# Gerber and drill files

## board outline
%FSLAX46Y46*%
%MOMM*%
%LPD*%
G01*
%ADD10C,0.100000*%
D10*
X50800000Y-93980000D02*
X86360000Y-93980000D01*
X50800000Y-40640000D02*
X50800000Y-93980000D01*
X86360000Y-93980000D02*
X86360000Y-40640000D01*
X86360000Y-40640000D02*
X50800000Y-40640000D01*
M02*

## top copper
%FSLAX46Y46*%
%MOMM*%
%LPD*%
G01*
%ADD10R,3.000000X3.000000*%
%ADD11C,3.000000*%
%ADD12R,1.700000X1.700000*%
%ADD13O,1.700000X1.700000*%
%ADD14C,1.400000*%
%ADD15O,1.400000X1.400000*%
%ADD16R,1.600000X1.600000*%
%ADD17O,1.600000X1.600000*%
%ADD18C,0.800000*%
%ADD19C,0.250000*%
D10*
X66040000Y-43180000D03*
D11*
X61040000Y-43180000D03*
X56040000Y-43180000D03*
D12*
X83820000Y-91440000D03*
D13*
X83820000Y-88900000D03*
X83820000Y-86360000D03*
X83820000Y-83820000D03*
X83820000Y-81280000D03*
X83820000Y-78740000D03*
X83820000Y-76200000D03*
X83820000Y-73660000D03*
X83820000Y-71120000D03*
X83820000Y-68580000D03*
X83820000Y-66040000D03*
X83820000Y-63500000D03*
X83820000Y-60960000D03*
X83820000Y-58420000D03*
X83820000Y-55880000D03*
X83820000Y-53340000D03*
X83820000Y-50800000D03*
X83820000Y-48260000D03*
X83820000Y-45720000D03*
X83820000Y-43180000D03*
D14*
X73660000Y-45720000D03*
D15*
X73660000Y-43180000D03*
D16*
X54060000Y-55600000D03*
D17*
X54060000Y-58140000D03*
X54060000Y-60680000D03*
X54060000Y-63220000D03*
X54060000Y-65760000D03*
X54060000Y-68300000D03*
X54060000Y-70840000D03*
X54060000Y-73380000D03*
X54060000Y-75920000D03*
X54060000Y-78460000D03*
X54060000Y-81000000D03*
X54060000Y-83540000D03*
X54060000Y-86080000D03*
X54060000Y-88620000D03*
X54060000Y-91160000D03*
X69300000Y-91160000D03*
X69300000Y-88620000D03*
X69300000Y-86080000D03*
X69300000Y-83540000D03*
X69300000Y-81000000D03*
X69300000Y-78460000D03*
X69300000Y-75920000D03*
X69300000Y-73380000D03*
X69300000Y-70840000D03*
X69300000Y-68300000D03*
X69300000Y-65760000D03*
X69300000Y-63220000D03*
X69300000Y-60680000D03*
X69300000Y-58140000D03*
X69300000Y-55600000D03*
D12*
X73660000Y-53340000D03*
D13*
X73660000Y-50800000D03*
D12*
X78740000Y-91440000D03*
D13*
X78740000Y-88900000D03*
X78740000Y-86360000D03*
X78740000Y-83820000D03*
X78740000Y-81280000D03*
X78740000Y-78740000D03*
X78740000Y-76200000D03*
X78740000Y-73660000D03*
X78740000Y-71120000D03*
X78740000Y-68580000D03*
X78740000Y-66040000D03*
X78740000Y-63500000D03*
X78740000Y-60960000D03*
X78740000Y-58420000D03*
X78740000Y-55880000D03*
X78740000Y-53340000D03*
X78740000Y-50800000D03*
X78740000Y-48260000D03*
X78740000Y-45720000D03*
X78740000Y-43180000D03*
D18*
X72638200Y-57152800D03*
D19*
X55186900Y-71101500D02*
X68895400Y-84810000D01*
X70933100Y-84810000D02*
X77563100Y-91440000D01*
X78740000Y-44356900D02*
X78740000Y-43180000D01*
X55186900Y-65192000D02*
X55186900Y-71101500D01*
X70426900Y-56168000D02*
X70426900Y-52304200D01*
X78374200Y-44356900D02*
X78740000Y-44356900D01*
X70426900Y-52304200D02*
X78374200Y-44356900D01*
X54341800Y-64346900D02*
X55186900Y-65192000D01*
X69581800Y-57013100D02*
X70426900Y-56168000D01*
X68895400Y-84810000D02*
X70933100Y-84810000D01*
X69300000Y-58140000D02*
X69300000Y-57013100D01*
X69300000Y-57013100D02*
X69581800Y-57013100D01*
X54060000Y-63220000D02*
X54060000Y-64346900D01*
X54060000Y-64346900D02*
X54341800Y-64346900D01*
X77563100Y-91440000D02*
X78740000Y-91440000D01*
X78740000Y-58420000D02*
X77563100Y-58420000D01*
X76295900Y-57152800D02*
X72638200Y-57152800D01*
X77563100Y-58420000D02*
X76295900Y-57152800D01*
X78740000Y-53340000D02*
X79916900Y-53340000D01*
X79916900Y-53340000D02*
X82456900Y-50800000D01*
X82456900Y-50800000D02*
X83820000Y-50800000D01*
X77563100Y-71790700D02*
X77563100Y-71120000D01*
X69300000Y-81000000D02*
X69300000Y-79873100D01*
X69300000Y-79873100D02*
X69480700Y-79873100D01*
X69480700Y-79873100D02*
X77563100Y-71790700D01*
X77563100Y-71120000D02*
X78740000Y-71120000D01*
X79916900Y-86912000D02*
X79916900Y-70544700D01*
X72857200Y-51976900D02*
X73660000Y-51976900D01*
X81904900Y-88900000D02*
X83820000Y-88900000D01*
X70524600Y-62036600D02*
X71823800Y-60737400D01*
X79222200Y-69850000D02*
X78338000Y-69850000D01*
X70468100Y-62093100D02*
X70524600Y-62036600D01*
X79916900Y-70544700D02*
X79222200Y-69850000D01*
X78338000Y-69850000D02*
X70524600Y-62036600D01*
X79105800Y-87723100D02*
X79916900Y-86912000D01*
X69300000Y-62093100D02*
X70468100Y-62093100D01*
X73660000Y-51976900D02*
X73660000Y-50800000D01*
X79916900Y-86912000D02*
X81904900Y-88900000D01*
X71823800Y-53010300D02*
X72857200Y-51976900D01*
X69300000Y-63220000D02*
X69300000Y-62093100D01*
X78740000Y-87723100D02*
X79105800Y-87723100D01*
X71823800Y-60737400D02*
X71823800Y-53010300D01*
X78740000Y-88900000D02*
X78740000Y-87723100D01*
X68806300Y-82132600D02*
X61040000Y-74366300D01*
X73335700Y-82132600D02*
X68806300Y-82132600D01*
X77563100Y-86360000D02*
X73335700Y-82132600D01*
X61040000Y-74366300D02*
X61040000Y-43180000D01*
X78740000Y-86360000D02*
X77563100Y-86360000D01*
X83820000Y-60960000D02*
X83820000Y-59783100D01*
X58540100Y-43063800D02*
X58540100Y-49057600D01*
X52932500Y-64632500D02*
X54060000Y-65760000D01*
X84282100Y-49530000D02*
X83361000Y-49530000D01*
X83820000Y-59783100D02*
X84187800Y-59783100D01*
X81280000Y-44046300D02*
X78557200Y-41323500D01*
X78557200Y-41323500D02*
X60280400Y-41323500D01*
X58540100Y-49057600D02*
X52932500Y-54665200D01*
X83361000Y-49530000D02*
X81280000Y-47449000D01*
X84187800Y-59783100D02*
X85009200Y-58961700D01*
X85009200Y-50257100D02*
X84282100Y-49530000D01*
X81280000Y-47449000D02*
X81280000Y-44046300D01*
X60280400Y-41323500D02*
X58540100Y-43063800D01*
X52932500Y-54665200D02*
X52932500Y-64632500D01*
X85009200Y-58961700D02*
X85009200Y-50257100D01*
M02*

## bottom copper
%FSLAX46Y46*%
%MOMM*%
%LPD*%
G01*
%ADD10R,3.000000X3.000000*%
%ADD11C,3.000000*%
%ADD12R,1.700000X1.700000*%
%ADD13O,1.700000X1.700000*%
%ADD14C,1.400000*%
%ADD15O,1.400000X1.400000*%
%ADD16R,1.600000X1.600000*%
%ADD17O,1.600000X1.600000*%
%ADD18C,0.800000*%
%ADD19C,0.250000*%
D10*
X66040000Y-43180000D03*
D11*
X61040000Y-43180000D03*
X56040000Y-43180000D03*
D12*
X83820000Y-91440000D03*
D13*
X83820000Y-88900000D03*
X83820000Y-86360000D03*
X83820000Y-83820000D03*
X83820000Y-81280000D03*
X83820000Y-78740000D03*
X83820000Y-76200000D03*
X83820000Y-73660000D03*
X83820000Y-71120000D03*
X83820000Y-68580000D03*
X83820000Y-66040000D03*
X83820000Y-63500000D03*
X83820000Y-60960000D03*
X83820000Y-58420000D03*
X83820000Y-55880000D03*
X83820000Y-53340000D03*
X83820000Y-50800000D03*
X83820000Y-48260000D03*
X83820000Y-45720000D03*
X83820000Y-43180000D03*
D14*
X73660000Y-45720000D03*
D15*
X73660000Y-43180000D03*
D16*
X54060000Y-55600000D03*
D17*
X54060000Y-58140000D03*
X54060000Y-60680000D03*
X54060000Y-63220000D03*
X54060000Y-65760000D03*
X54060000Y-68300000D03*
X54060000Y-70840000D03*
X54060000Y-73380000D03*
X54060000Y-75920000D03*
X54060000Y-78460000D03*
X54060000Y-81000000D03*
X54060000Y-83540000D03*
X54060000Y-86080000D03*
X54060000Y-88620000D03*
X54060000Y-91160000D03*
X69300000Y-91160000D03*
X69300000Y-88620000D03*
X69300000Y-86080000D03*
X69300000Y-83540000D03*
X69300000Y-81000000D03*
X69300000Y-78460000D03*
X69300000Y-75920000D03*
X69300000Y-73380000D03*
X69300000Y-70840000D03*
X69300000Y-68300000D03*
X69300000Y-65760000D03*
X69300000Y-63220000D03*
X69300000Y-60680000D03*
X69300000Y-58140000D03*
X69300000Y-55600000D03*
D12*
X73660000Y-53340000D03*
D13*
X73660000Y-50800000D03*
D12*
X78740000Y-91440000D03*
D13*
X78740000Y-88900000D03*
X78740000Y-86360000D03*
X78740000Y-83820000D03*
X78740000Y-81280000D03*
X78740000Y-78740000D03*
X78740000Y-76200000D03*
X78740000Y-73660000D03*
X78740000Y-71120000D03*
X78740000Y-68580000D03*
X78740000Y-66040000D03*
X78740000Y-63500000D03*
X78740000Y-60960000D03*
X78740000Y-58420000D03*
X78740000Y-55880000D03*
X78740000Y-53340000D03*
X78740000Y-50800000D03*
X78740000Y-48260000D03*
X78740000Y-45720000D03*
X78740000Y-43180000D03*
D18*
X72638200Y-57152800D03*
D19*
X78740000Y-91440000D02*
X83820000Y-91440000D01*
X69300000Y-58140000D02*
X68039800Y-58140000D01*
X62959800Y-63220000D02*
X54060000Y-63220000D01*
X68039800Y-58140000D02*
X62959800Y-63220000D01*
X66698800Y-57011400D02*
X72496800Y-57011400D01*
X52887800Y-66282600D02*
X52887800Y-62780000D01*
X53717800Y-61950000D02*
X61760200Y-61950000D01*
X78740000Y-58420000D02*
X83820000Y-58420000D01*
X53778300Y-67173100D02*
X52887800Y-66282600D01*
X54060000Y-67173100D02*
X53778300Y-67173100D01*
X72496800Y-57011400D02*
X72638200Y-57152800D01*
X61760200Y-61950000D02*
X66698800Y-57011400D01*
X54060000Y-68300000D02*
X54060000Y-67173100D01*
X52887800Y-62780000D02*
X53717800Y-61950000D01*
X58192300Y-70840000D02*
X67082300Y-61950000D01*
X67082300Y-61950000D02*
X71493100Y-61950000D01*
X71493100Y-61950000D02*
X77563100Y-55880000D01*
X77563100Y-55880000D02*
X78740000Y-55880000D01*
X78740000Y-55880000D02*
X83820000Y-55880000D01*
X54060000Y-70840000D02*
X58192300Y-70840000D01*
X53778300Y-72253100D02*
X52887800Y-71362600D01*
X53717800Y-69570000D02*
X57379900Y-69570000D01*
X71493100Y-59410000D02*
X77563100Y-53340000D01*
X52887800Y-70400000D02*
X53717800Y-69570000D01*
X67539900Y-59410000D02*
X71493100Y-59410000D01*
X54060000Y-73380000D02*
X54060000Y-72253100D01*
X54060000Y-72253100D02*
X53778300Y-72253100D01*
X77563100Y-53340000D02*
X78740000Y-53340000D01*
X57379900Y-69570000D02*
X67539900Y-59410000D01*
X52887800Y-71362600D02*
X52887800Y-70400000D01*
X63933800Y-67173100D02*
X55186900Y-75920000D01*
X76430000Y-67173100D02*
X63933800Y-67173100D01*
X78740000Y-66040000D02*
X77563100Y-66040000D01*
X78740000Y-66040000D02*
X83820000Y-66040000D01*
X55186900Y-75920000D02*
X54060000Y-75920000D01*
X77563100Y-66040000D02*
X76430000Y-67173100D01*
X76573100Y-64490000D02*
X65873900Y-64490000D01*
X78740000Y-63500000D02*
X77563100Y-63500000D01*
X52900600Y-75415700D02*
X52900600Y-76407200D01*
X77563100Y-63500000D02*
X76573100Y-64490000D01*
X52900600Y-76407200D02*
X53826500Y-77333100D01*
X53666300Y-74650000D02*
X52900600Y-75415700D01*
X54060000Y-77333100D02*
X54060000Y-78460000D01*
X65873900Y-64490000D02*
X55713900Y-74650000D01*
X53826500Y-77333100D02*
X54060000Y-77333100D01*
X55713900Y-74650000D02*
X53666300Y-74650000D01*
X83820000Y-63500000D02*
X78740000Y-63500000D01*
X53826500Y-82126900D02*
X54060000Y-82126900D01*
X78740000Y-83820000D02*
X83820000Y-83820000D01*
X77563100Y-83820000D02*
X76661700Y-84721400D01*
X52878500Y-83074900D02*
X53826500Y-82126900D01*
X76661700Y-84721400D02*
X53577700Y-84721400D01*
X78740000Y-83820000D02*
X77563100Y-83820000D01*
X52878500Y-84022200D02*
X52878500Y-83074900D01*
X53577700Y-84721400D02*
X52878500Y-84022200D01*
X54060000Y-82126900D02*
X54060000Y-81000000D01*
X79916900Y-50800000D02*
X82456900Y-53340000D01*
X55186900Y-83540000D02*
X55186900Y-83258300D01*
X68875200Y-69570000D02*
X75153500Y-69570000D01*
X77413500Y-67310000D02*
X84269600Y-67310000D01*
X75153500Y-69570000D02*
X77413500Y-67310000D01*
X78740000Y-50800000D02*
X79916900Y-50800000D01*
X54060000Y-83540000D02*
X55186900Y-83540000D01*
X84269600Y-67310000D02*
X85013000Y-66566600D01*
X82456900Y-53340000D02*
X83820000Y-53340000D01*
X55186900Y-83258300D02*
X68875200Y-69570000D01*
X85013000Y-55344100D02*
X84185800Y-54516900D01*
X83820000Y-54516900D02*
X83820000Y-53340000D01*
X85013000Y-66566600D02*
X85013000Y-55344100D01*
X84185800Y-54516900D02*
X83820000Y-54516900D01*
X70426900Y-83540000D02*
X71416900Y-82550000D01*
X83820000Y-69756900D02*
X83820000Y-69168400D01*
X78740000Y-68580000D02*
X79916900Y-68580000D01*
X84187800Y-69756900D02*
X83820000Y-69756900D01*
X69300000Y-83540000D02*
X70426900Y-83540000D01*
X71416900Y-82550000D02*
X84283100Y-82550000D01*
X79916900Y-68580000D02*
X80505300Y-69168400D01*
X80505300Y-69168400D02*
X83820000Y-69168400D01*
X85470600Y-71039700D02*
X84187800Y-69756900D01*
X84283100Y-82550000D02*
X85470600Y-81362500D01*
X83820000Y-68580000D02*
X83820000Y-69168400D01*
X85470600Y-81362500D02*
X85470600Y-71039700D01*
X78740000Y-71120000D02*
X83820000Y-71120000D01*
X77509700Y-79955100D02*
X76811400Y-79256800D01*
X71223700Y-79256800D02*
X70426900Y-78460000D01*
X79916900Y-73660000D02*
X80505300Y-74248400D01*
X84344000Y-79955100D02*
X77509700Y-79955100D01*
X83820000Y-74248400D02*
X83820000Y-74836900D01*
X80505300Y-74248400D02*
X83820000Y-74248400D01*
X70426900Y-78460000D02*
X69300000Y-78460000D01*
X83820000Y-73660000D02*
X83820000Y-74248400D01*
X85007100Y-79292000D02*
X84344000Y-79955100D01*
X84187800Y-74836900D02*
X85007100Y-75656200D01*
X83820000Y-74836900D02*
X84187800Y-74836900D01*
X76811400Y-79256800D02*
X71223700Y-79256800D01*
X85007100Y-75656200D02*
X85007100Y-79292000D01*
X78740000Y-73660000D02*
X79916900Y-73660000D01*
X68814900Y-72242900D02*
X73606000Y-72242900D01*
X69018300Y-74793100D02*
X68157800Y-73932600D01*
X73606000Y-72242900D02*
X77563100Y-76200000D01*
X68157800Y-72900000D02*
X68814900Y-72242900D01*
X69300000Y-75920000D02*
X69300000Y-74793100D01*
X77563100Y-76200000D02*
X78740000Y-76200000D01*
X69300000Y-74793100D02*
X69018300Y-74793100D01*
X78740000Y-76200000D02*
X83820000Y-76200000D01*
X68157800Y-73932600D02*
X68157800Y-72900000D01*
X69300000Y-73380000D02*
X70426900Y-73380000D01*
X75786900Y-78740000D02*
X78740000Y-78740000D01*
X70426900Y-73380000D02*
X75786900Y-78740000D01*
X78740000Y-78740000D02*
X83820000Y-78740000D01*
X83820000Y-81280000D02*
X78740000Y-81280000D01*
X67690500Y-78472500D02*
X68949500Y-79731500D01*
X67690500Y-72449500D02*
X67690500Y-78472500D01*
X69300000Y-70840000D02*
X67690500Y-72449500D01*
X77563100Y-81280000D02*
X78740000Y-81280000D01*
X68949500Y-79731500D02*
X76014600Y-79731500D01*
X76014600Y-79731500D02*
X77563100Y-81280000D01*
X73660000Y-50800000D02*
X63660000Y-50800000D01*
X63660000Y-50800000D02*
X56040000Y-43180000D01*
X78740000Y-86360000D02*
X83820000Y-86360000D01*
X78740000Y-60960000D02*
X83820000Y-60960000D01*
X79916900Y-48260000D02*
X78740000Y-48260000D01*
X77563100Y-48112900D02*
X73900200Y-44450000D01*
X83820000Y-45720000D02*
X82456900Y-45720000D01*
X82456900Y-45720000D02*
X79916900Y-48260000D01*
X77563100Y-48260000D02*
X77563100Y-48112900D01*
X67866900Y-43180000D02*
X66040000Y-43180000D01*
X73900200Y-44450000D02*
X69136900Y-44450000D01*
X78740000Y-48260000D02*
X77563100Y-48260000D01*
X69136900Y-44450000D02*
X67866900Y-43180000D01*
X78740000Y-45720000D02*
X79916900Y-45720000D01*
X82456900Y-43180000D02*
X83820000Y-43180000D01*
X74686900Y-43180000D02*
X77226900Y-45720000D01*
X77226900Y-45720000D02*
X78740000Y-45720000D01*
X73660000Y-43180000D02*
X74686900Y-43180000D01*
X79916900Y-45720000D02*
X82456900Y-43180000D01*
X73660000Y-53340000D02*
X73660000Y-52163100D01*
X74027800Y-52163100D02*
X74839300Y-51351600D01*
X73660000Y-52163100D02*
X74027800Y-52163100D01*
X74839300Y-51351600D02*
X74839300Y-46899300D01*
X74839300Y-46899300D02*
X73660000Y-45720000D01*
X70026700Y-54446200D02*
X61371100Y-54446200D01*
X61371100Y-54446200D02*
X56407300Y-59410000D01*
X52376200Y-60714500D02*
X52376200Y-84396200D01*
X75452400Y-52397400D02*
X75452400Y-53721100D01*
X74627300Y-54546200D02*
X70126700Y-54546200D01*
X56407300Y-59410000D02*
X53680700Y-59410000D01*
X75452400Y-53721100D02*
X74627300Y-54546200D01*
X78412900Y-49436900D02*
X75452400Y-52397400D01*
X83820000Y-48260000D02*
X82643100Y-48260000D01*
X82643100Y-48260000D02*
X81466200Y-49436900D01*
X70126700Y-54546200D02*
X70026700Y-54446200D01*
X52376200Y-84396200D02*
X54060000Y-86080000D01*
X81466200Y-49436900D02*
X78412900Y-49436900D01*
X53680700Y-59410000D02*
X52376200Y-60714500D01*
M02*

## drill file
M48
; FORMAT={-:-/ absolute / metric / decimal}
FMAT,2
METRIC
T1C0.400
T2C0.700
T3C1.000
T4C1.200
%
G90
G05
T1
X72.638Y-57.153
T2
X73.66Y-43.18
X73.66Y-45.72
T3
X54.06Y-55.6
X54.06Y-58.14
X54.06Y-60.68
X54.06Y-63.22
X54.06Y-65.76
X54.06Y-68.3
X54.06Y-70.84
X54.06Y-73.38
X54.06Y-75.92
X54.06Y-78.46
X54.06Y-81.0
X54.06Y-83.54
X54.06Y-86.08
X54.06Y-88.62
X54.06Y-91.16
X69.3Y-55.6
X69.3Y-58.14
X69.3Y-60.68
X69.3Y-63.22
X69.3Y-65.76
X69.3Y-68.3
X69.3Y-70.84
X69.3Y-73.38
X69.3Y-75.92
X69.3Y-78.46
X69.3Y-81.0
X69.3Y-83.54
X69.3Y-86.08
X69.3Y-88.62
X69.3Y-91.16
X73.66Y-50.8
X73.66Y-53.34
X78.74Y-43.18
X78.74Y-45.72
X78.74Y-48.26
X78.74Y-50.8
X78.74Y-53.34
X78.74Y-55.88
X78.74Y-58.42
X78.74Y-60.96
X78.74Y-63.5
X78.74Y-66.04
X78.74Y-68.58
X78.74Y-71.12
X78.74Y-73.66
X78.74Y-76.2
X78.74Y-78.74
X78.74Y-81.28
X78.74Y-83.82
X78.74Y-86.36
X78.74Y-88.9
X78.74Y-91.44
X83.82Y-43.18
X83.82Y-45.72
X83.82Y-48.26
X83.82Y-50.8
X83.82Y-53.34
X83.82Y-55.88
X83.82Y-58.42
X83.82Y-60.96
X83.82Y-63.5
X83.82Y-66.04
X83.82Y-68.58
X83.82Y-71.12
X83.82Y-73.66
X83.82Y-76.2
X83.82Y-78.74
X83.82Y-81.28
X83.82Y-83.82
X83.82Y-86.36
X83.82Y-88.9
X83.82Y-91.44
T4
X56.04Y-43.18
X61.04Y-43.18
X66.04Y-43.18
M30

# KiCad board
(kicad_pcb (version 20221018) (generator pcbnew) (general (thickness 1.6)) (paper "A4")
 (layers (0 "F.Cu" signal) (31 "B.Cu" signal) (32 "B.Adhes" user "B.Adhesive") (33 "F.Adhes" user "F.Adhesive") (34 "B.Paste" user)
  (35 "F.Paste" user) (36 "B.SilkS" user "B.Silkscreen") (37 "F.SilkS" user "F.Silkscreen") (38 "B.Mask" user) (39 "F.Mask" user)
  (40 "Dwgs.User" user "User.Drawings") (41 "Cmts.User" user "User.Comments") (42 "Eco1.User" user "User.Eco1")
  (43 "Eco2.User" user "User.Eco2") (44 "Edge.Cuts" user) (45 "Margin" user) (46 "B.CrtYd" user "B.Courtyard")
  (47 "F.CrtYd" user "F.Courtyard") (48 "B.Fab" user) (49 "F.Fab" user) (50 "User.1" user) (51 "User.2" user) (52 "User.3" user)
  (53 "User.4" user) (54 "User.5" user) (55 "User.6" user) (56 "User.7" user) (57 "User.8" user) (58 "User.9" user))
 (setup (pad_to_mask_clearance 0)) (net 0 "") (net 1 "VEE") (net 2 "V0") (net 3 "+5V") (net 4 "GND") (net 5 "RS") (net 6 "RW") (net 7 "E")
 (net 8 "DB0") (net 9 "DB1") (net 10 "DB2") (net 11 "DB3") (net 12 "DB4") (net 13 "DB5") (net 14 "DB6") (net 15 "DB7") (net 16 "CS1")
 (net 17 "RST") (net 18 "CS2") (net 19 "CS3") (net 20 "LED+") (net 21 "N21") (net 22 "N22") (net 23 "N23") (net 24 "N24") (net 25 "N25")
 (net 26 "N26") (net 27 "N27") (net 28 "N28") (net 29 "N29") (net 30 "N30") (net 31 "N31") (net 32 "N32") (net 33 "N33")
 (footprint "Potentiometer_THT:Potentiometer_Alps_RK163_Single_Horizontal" (layer "F.Cu") (at 66.04 43.18 -90)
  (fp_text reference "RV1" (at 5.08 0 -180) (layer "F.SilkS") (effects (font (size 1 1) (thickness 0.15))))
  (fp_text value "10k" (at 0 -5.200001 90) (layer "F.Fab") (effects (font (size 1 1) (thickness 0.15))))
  (pad "1" thru_hole rect (at 0 0 90) (size 3 3) (drill 1.2) (layers "*.Cu" "*.Mask") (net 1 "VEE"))
  (pad "2" thru_hole circle (at 0 5 90) (size 3 3) (drill 1.2) (layers "*.Cu" "*.Mask") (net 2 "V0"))
  (pad "3" thru_hole circle (at 0 10 90) (size 3 3) (drill 1.2) (layers "*.Cu" "*.Mask") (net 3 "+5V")))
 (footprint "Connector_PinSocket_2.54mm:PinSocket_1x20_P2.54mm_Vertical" (layer "F.Cu") (at 83.82 91.44 180)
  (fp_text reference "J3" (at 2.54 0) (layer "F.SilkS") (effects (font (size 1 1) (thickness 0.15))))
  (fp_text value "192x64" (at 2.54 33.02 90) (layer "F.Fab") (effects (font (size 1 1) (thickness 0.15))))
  (pad "1" thru_hole rect (at 0 0 180) (size 1.7 1.7) (drill 1) (layers "*.Cu" "*.Mask") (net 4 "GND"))
  (pad "2" thru_hole oval (at 0 2.54 180) (size 1.7 1.7) (drill 1) (layers "*.Cu" "*.Mask") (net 3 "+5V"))
  (pad "3" thru_hole oval (at 0 5.08 180) (size 1.7 1.7) (drill 1) (layers "*.Cu" "*.Mask") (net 2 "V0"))
  (pad "4" thru_hole oval (at 0 7.62 180) (size 1.7 1.7) (drill 1) (layers "*.Cu" "*.Mask") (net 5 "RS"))
  (pad "5" thru_hole oval (at 0 10.16 180) (size 1.7 1.7) (drill 1) (layers "*.Cu" "*.Mask") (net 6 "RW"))
  (pad "6" thru_hole oval (at 0 12.7 180) (size 1.7 1.7) (drill 1) (layers "*.Cu" "*.Mask") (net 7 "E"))
  (pad "7" thru_hole oval (at 0 15.24 180) (size 1.7 1.7) (drill 1) (layers "*.Cu" "*.Mask") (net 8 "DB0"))
  (pad "8" thru_hole oval (at 0 17.78 180) (size 1.7 1.7) (drill 1) (layers "*.Cu" "*.Mask") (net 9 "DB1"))
  (pad "9" thru_hole oval (at 0 20.32 180) (size 1.7 1.7) (drill 1) (layers "*.Cu" "*.Mask") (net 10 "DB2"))
  (pad "10" thru_hole oval (at 0 22.86 180) (size 1.7 1.7) (drill 1) (layers "*.Cu" "*.Mask") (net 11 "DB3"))
  (pad "11" thru_hole oval (at 0 25.4 180) (size 1.7 1.7) (drill 1) (layers "*.Cu" "*.Mask") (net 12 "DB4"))
  (pad "12" thru_hole oval (at 0 27.94 180) (size 1.7 1.7) (drill 1) (layers "*.Cu" "*.Mask") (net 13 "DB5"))
  (pad "13" thru_hole oval (at 0 30.48 180) (size 1.7 1.7) (drill 1) (layers "*.Cu" "*.Mask") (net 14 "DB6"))
  (pad "14" thru_hole oval (at 0 33.02 180) (size 1.7 1.7) (drill 1) (layers "*.Cu" "*.Mask") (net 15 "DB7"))
  (pad "15" thru_hole oval (at 0 35.56 180) (size 1.7 1.7) (drill 1) (layers "*.Cu" "*.Mask") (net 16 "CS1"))
  (pad "16" thru_hole oval (at 0 38.1 180) (size 1.7 1.7) (drill 1) (layers "*.Cu" "*.Mask") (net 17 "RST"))
  (pad "17" thru_hole oval (at 0 40.64 180) (size 1.7 1.7) (drill 1) (layers "*.Cu" "*.Mask") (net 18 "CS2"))
  (pad "18" thru_hole oval (at 0 43.18 180) (size 1.7 1.7) (drill 1) (layers "*.Cu" "*.Mask") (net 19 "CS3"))
  (pad "19" thru_hole oval (at 0 45.72 180) (size 1.7 1.7) (drill 1) (layers "*.Cu" "*.Mask") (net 1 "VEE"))
  (pad "20" thru_hole oval (at 0 48.26 180) (size 1.7 1.7) (drill 1) (layers "*.Cu" "*.Mask") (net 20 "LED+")))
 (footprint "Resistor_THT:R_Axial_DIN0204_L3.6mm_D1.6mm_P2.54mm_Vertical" (layer "F.Cu") (at 73.66 45.72 90)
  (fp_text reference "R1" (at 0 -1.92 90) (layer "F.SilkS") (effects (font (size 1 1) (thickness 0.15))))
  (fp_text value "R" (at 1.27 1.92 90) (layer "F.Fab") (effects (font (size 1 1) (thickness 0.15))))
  (pad "1" thru_hole circle (at 0 0 90) (size 1.4 1.4) (drill 0.7) (layers "*.Cu" "*.Mask") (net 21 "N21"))
  (pad "2" thru_hole oval (at 2.54 0 90) (size 1.4 1.4) (drill 0.7) (layers "*.Cu" "*.Mask") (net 20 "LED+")))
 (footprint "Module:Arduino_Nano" (layer "F.Cu") (at 54.06 55.6)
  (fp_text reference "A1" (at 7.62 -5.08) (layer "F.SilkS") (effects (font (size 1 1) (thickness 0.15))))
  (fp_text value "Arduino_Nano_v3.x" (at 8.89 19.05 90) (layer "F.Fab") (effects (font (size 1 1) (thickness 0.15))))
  (pad "1" thru_hole rect (at 0 0) (size 1.6 1.6) (drill 1) (layers "*.Cu" "*.Mask") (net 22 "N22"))
  (pad "2" thru_hole oval (at 0 2.54) (size 1.6 1.6) (drill 1) (layers "*.Cu" "*.Mask") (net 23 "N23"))
  (pad "3" thru_hole oval (at 0 5.08) (size 1.6 1.6) (drill 1) (layers "*.Cu" "*.Mask") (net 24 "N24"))
  (pad "4" thru_hole oval (at 0 7.62) (size 1.6 1.6) (drill 1) (layers "*.Cu" "*.Mask") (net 4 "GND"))
  (pad "5" thru_hole oval (at 0 10.16) (size 1.6 1.6) (drill 1) (layers "*.Cu" "*.Mask") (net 14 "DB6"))
  (pad "6" thru_hole oval (at 0 12.7) (size 1.6 1.6) (drill 1) (layers "*.Cu" "*.Mask") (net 15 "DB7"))
  (pad "7" thru_hole oval (at 0 15.24) (size 1.6 1.6) (drill 1) (layers "*.Cu" "*.Mask") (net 16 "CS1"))
  (pad "8" thru_hole oval (at 0 17.78) (size 1.6 1.6) (drill 1) (layers "*.Cu" "*.Mask") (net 18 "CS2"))
  (pad "9" thru_hole oval (at 0 20.32) (size 1.6 1.6) (drill 1) (layers "*.Cu" "*.Mask") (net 12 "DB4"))
  (pad "10" thru_hole oval (at 0 22.86) (size 1.6 1.6) (drill 1) (layers "*.Cu" "*.Mask") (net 13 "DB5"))
  (pad "11" thru_hole oval (at 0 25.4) (size 1.6 1.6) (drill 1) (layers "*.Cu" "*.Mask") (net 5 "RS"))
  (pad "12" thru_hole oval (at 0 27.94) (size 1.6 1.6) (drill 1) (layers "*.Cu" "*.Mask") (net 17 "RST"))
  (pad "13" thru_hole oval (at 0 30.48) (size 1.6 1.6) (drill 1) (layers "*.Cu" "*.Mask") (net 19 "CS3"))
  (pad "14" thru_hole oval (at 0 33.02) (size 1.6 1.6) (drill 1) (layers "*.Cu" "*.Mask") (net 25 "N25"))
  (pad "15" thru_hole oval (at 0 35.56) (size 1.6 1.6) (drill 1) (layers "*.Cu" "*.Mask") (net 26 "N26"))
  (pad "16" thru_hole oval (at 15.24 35.56) (size 1.6 1.6) (drill 1) (layers "*.Cu" "*.Mask") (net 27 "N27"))
  (pad "17" thru_hole oval (at 15.24 33.02) (size 1.6 1.6) (drill 1) (layers "*.Cu" "*.Mask") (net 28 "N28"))
  (pad "18" thru_hole oval (at 15.24 30.48) (size 1.6 1.6) (drill 1) (layers "*.Cu" "*.Mask") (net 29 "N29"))
  (pad "19" thru_hole oval (at 15.24 27.94) (size 1.6 1.6) (drill 1) (layers "*.Cu" "*.Mask") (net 11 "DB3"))
  (pad "20" thru_hole oval (at 15.24 25.4) (size 1.6 1.6) (drill 1) (layers "*.Cu" "*.Mask") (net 10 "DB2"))
  (pad "21" thru_hole oval (at 15.24 22.86) (size 1.6 1.6) (drill 1) (layers "*.Cu" "*.Mask") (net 9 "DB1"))
  (pad "22" thru_hole oval (at 15.24 20.32) (size 1.6 1.6) (drill 1) (layers "*.Cu" "*.Mask") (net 8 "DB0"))
  (pad "23" thru_hole oval (at 15.24 17.78) (size 1.6 1.6) (drill 1) (layers "*.Cu" "*.Mask") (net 7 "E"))
  (pad "24" thru_hole oval (at 15.24 15.24) (size 1.6 1.6) (drill 1) (layers "*.Cu" "*.Mask") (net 6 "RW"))
  (pad "25" thru_hole oval (at 15.24 12.7) (size 1.6 1.6) (drill 1) (layers "*.Cu" "*.Mask") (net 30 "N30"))
  (pad "26" thru_hole oval (at 15.24 10.16) (size 1.6 1.6) (drill 1) (layers "*.Cu" "*.Mask") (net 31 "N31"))
  (pad "27" thru_hole oval (at 15.24 7.62) (size 1.6 1.6) (drill 1) (layers "*.Cu" "*.Mask") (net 3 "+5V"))
  (pad "28" thru_hole oval (at 15.24 5.08) (size 1.6 1.6) (drill 1) (layers "*.Cu" "*.Mask") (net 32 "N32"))
  (pad "29" thru_hole oval (at 15.24 2.54) (size 1.6 1.6) (drill 1) (layers "*.Cu" "*.Mask") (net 4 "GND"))
  (pad "30" thru_hole oval (at 15.24 0) (size 1.6 1.6) (drill 1) (layers "*.Cu" "*.Mask") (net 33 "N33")))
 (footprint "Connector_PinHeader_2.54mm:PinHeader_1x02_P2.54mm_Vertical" (layer "F.Cu") (at 73.66 53.34 180)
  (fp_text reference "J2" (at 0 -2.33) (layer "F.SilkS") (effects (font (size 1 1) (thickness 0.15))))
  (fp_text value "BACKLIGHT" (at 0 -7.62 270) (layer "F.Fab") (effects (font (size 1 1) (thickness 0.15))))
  (pad "1" thru_hole rect (at 0 0 180) (size 1.7 1.7) (drill 1) (layers "*.Cu" "*.Mask") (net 21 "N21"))
  (pad "2" thru_hole oval (at 0 2.54 180) (size 1.7 1.7) (drill 1) (layers "*.Cu" "*.Mask") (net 3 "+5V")))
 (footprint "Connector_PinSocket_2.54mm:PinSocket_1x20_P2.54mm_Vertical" (layer "F.Cu") (at 78.74 91.44 180)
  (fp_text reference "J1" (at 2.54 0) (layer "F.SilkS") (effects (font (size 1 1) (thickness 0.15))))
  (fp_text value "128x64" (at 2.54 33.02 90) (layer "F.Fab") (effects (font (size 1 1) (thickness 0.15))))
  (pad "1" thru_hole rect (at 0 0 180) (size 1.7 1.7) (drill 1) (layers "*.Cu" "*.Mask") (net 4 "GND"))
  (pad "2" thru_hole oval (at 0 2.54 180) (size 1.7 1.7) (drill 1) (layers "*.Cu" "*.Mask") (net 3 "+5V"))
  (pad "3" thru_hole oval (at 0 5.08 180) (size 1.7 1.7) (drill 1) (layers "*.Cu" "*.Mask") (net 2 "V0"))
  (pad "4" thru_hole oval (at 0 7.62 180) (size 1.7 1.7) (drill 1) (layers "*.Cu" "*.Mask") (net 5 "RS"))
  (pad "5" thru_hole oval (at 0 10.16 180) (size 1.7 1.7) (drill 1) (layers "*.Cu" "*.Mask") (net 6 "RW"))
  (pad "6" thru_hole oval (at 0 12.7 180) (size 1.7 1.7) (drill 1) (layers "*.Cu" "*.Mask") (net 7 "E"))
  (pad "7" thru_hole oval (at 0 15.24 180) (size 1.7 1.7) (drill 1) (layers "*.Cu" "*.Mask") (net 8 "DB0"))
  (pad "8" thru_hole oval (at 0 17.78 180) (size 1.7 1.7) (drill 1) (layers "*.Cu" "*.Mask") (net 9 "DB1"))
  (pad "9" thru_hole oval (at 0 20.32 180) (size 1.7 1.7) (drill 1) (layers "*.Cu" "*.Mask") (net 10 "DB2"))
  (pad "10" thru_hole oval (at 0 22.86 180) (size 1.7 1.7) (drill 1) (layers "*.Cu" "*.Mask") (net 11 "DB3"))
  (pad "11" thru_hole oval (at 0 25.4 180) (size 1.7 1.7) (drill 1) (layers "*.Cu" "*.Mask") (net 12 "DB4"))
  (pad "12" thru_hole oval (at 0 27.94 180) (size 1.7 1.7) (drill 1) (layers "*.Cu" "*.Mask") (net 13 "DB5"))
  (pad "13" thru_hole oval (at 0 30.48 180) (size 1.7 1.7) (drill 1) (layers "*.Cu" "*.Mask") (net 14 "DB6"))
  (pad "14" thru_hole oval (at 0 33.02 180) (size 1.7 1.7) (drill 1) (layers "*.Cu" "*.Mask") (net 15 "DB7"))
  (pad "15" thru_hole oval (at 0 35.56 180) (size 1.7 1.7) (drill 1) (layers "*.Cu" "*.Mask") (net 16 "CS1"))
  (pad "16" thru_hole oval (at 0 38.1 180) (size 1.7 1.7) (drill 1) (layers "*.Cu" "*.Mask") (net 18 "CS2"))
  (pad "17" thru_hole oval (at 0 40.64 180) (size 1.7 1.7) (drill 1) (layers "*.Cu" "*.Mask") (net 17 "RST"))
  (pad "18" thru_hole oval (at 0 43.18 180) (size 1.7 1.7) (drill 1) (layers "*.Cu" "*.Mask") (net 1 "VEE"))
  (pad "19" thru_hole oval (at 0 45.72 180) (size 1.7 1.7) (drill 1) (layers "*.Cu" "*.Mask") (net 20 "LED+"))
  (pad "20" thru_hole oval (at 0 48.26 180) (size 1.7 1.7) (drill 1) (layers "*.Cu" "*.Mask") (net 4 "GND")))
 (gr_line (start 50.8 93.98) (end 86.36 93.98) (stroke (width 0.1) (type default)) (layer "Edge.Cuts"))
 (gr_line (start 50.8 40.64) (end 50.8 93.98) (stroke (width 0.1) (type default)) (layer "Edge.Cuts"))
 (gr_line (start 86.36 93.98) (end 86.36 40.64) (stroke (width 0.1) (type default)) (layer "Edge.Cuts"))
 (gr_line (start 86.36 40.64) (end 50.8 40.64) (stroke (width 0.1) (type default)) (layer "Edge.Cuts"))
 (segment (start 55.1869 71.1015) (end 68.8954 84.81) (width 0.25) (layer "F.Cu") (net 4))
 (segment (start 70.9331 84.81) (end 77.5631 91.44) (width 0.25) (layer "F.Cu") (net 4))
 (segment (start 78.74 44.3569) (end 78.74 43.18) (width 0.25) (layer "F.Cu") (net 4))
 (segment (start 55.1869 65.192) (end 55.1869 71.1015) (width 0.25) (layer "F.Cu") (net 4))
 (segment (start 70.4269 56.168) (end 70.4269 52.3042) (width 0.25) (layer "F.Cu") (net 4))
 (segment (start 78.3742 44.3569) (end 78.74 44.3569) (width 0.25) (layer "F.Cu") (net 4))
 (segment (start 70.4269 52.3042) (end 78.3742 44.3569) (width 0.25) (layer "F.Cu") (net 4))
 (segment (start 54.3418 64.3469) (end 55.1869 65.192) (width 0.25) (layer "F.Cu") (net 4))
 (segment (start 69.5818 57.0131) (end 70.4269 56.168) (width 0.25) (layer "F.Cu") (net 4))
 (segment (start 68.8954 84.81) (end 70.9331 84.81) (width 0.25) (layer "F.Cu") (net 4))
 (segment (start 69.3 58.14) (end 69.3 57.0131) (width 0.25) (layer "F.Cu") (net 4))
 (segment (start 69.3 57.0131) (end 69.5818 57.0131) (width 0.25) (layer "F.Cu") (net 4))
 (segment (start 54.06 63.22) (end 54.06 64.3469) (width 0.25) (layer "F.Cu") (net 4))
 (segment (start 54.06 64.3469) (end 54.3418 64.3469) (width 0.25) (layer "F.Cu") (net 4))
 (segment (start 77.5631 91.44) (end 78.74 91.44) (width 0.25) (layer "F.Cu") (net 4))
 (segment (start 78.74 91.44) (end 83.82 91.44) (width 0.25) (layer "B.Cu") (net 4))
 (segment (start 69.3 58.14) (end 68.0398 58.14) (width 0.25) (layer "B.Cu") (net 4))
 (segment (start 62.9598 63.22) (end 54.06 63.22) (width 0.25) (layer "B.Cu") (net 4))
 (segment (start 68.0398 58.14) (end 62.9598 63.22) (width 0.25) (layer "B.Cu") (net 4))
 (segment (start 78.74 58.42) (end 77.5631 58.42) (width 0.25) (layer "F.Cu") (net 15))
 (segment (start 76.2959 57.1528) (end 72.6382 57.1528) (width 0.25) (layer "F.Cu") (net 15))
 (segment (start 77.5631 58.42) (end 76.2959 57.1528) (width 0.25) (layer "F.Cu") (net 15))
 (via (at 72.6382 57.1528) (size 0.8) (drill 0.4) (layers "F.Cu" "B.Cu") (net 15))
 (segment (start 66.6988 57.0114) (end 72.4968 57.0114) (width 0.25) (layer "B.Cu") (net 15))
 (segment (start 52.8878 66.2826) (end 52.8878 62.78) (width 0.25) (layer "B.Cu") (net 15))
 (segment (start 53.7178 61.95) (end 61.7602 61.95) (width 0.25) (layer "B.Cu") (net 15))
 (segment (start 78.74 58.42) (end 83.82 58.42) (width 0.25) (layer "B.Cu") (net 15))
 (segment (start 53.7783 67.1731) (end 52.8878 66.2826) (width 0.25) (layer "B.Cu") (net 15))
 (segment (start 54.06 67.1731) (end 53.7783 67.1731) (width 0.25) (layer "B.Cu") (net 15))
 (segment (start 72.4968 57.0114) (end 72.6382 57.1528) (width 0.25) (layer "B.Cu") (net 15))
 (segment (start 61.7602 61.95) (end 66.6988 57.0114) (width 0.25) (layer "B.Cu") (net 15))
 (segment (start 54.06 68.3) (end 54.06 67.1731) (width 0.25) (layer "B.Cu") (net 15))
 (segment (start 52.8878 62.78) (end 53.7178 61.95) (width 0.25) (layer "B.Cu") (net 15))
 (segment (start 58.1923 70.84) (end 67.0823 61.95) (width 0.25) (layer "B.Cu") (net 16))
 (segment (start 67.0823 61.95) (end 71.4931 61.95) (width 0.25) (layer "B.Cu") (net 16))
 (segment (start 71.4931 61.95) (end 77.5631 55.88) (width 0.25) (layer "B.Cu") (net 16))
 (segment (start 77.5631 55.88) (end 78.74 55.88) (width 0.25) (layer "B.Cu") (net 16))
 (segment (start 78.74 55.88) (end 83.82 55.88) (width 0.25) (layer "B.Cu") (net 16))
 (segment (start 54.06 70.84) (end 58.1923 70.84) (width 0.25) (layer "B.Cu") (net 16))
 (segment (start 78.74 53.34) (end 79.9169 53.34) (width 0.25) (layer "F.Cu") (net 18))
 (segment (start 79.9169 53.34) (end 82.4569 50.8) (width 0.25) (layer "F.Cu") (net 18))
 (segment (start 82.4569 50.8) (end 83.82 50.8) (width 0.25) (layer "F.Cu") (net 18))
 (segment (start 53.7783 72.2531) (end 52.8878 71.3626) (width 0.25) (layer "B.Cu") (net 18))
 (segment (start 53.7178 69.57) (end 57.3799 69.57) (width 0.25) (layer "B.Cu") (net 18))
 (segment (start 71.4931 59.41) (end 77.5631 53.34) (width 0.25) (layer "B.Cu") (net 18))
 (segment (start 52.8878 70.4) (end 53.7178 69.57) (width 0.25) (layer "B.Cu") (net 18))
 (segment (start 67.5399 59.41) (end 71.4931 59.41) (width 0.25) (layer "B.Cu") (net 18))
 (segment (start 54.06 73.38) (end 54.06 72.2531) (width 0.25) (layer "B.Cu") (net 18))
 (segment (start 54.06 72.2531) (end 53.7783 72.2531) (width 0.25) (layer "B.Cu") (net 18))
 (segment (start 77.5631 53.34) (end 78.74 53.34) (width 0.25) (layer "B.Cu") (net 18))
 (segment (start 57.3799 69.57) (end 67.5399 59.41) (width 0.25) (layer "B.Cu") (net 18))
 (segment (start 52.8878 71.3626) (end 52.8878 70.4) (width 0.25) (layer "B.Cu") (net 18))
 (segment (start 63.9338 67.1731) (end 55.1869 75.92) (width 0.25) (layer "B.Cu") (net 12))
 (segment (start 76.43 67.1731) (end 63.9338 67.1731) (width 0.25) (layer "B.Cu") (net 12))
 (segment (start 78.74 66.04) (end 77.5631 66.04) (width 0.25) (layer "B.Cu") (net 12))
 (segment (start 78.74 66.04) (end 83.82 66.04) (width 0.25) (layer "B.Cu") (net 12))
 (segment (start 55.1869 75.92) (end 54.06 75.92) (width 0.25) (layer "B.Cu") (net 12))
 (segment (start 77.5631 66.04) (end 76.43 67.1731) (width 0.25) (layer "B.Cu") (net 12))
 (segment (start 76.5731 64.49) (end 65.8739 64.49) (width 0.25) (layer "B.Cu") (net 13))
 (segment (start 78.74 63.5) (end 77.5631 63.5) (width 0.25) (layer "B.Cu") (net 13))
 (segment (start 52.9006 75.4157) (end 52.9006 76.4072) (width 0.25) (layer "B.Cu") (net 13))
 (segment (start 77.5631 63.5) (end 76.5731 64.49) (width 0.25) (layer "B.Cu") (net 13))
 (segment (start 52.9006 76.4072) (end 53.8265 77.3331) (width 0.25) (layer "B.Cu") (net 13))
 (segment (start 53.6663 74.65) (end 52.9006 75.4157) (width 0.25) (layer "B.Cu") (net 13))
 (segment (start 54.06 77.3331) (end 54.06 78.46) (width 0.25) (layer "B.Cu") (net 13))
 (segment (start 65.8739 64.49) (end 55.7139 74.65) (width 0.25) (layer "B.Cu") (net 13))
 (segment (start 53.8265 77.3331) (end 54.06 77.3331) (width 0.25) (layer "B.Cu") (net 13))
 (segment (start 55.7139 74.65) (end 53.6663 74.65) (width 0.25) (layer "B.Cu") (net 13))
 (segment (start 83.82 63.5) (end 78.74 63.5) (width 0.25) (layer "B.Cu") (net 13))
 (segment (start 53.8265 82.1269) (end 54.06 82.1269) (width 0.25) (layer "B.Cu") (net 5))
 (segment (start 78.74 83.82) (end 83.82 83.82) (width 0.25) (layer "B.Cu") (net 5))
 (segment (start 77.5631 83.82) (end 76.6617 84.7214) (width 0.25) (layer "B.Cu") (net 5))
 (segment (start 52.8785 83.0749) (end 53.8265 82.1269) (width 0.25) (layer "B.Cu") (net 5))
 (segment (start 76.6617 84.7214) (end 53.5777 84.7214) (width 0.25) (layer "B.Cu") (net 5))
 (segment (start 78.74 83.82) (end 77.5631 83.82) (width 0.25) (layer "B.Cu") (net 5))
 (segment (start 52.8785 84.0222) (end 52.8785 83.0749) (width 0.25) (layer "B.Cu") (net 5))
 (segment (start 53.5777 84.7214) (end 52.8785 84.0222) (width 0.25) (layer "B.Cu") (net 5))
 (segment (start 54.06 82.1269) (end 54.06 81) (width 0.25) (layer "B.Cu") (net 5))
 (segment (start 79.9169 50.8) (end 82.4569 53.34) (width 0.25) (layer "B.Cu") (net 17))
 (segment (start 55.1869 83.54) (end 55.1869 83.2583) (width 0.25) (layer "B.Cu") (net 17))
 (segment (start 68.8752 69.57) (end 75.1535 69.57) (width 0.25) (layer "B.Cu") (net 17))
 (segment (start 77.4135 67.31) (end 84.2696 67.31) (width 0.25) (layer "B.Cu") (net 17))
 (segment (start 75.1535 69.57) (end 77.4135 67.31) (width 0.25) (layer "B.Cu") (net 17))
 (segment (start 78.74 50.8) (end 79.9169 50.8) (width 0.25) (layer "B.Cu") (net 17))
 (segment (start 54.06 83.54) (end 55.1869 83.54) (width 0.25) (layer "B.Cu") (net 17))
 (segment (start 84.2696 67.31) (end 85.013 66.5666) (width 0.25) (layer "B.Cu") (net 17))
 (segment (start 82.4569 53.34) (end 83.82 53.34) (width 0.25) (layer "B.Cu") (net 17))
 (segment (start 55.1869 83.2583) (end 68.8752 69.57) (width 0.25) (layer "B.Cu") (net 17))
 (segment (start 85.013 55.3441) (end 84.1858 54.5169) (width 0.25) (layer "B.Cu") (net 17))
 (segment (start 83.82 54.5169) (end 83.82 53.34) (width 0.25) (layer "B.Cu") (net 17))
 (segment (start 85.013 66.5666) (end 85.013 55.3441) (width 0.25) (layer "B.Cu") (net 17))
 (segment (start 84.1858 54.5169) (end 83.82 54.5169) (width 0.25) (layer "B.Cu") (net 17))
 (segment (start 70.4269 83.54) (end 71.4169 82.55) (width 0.25) (layer "B.Cu") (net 11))
 (segment (start 83.82 69.7569) (end 83.82 69.1684) (width 0.25) (layer "B.Cu") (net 11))
 (segment (start 78.74 68.58) (end 79.9169 68.58) (width 0.25) (layer "B.Cu") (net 11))
 (segment (start 84.1878 69.7569) (end 83.82 69.7569) (width 0.25) (layer "B.Cu") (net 11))
 (segment (start 69.3 83.54) (end 70.4269 83.54) (width 0.25) (layer "B.Cu") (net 11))
 (segment (start 71.4169 82.55) (end 84.2831 82.55) (width 0.25) (layer "B.Cu") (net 11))
 (segment (start 79.9169 68.58) (end 80.5053 69.1684) (width 0.25) (layer "B.Cu") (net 11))
 (segment (start 80.5053 69.1684) (end 83.82 69.1684) (width 0.25) (layer "B.Cu") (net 11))
 (segment (start 85.4706 71.0397) (end 84.1878 69.7569) (width 0.25) (layer "B.Cu") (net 11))
 (segment (start 84.2831 82.55) (end 85.4706 81.3625) (width 0.25) (layer "B.Cu") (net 11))
 (segment (start 83.82 68.58) (end 83.82 69.1684) (width 0.25) (layer "B.Cu") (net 11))
 (segment (start 85.4706 81.3625) (end 85.4706 71.0397) (width 0.25) (layer "B.Cu") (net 11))
 (segment (start 77.5631 71.7907) (end 77.5631 71.12) (width 0.25) (layer "F.Cu") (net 10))
 (segment (start 69.3 81) (end 69.3 79.8731) (width 0.25) (layer "F.Cu") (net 10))
 (segment (start 69.3 79.8731) (end 69.4807 79.8731) (width 0.25) (layer "F.Cu") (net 10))
 (segment (start 69.4807 79.8731) (end 77.5631 71.7907) (width 0.25) (layer "F.Cu") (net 10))
 (segment (start 77.5631 71.12) (end 78.74 71.12) (width 0.25) (layer "F.Cu") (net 10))
 (segment (start 78.74 71.12) (end 83.82 71.12) (width 0.25) (layer "B.Cu") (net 10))
 (segment (start 77.5097 79.9551) (end 76.8114 79.2568) (width 0.25) (layer "B.Cu") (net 9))
 (segment (start 71.2237 79.2568) (end 70.4269 78.46) (width 0.25) (layer "B.Cu") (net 9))
 (segment (start 79.9169 73.66) (end 80.5053 74.2484) (width 0.25) (layer "B.Cu") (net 9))
 (segment (start 84.344 79.9551) (end 77.5097 79.9551) (width 0.25) (layer "B.Cu") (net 9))
 (segment (start 83.82 74.2484) (end 83.82 74.8369) (width 0.25) (layer "B.Cu") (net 9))
 (segment (start 80.5053 74.2484) (end 83.82 74.2484) (width 0.25) (layer "B.Cu") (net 9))
 (segment (start 70.4269 78.46) (end 69.3 78.46) (width 0.25) (layer "B.Cu") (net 9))
 (segment (start 83.82 73.66) (end 83.82 74.2484) (width 0.25) (layer "B.Cu") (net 9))
 (segment (start 85.0071 79.292) (end 84.344 79.9551) (width 0.25) (layer "B.Cu") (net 9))
 (segment (start 84.1878 74.8369) (end 85.0071 75.6562) (width 0.25) (layer "B.Cu") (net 9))
 (segment (start 83.82 74.8369) (end 84.1878 74.8369) (width 0.25) (layer "B.Cu") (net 9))
 (segment (start 76.8114 79.2568) (end 71.2237 79.2568) (width 0.25) (layer "B.Cu") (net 9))
 (segment (start 85.0071 75.6562) (end 85.0071 79.292) (width 0.25) (layer "B.Cu") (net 9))
 (segment (start 78.74 73.66) (end 79.9169 73.66) (width 0.25) (layer "B.Cu") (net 9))
 (segment (start 68.8149 72.2429) (end 73.606 72.2429) (width 0.25) (layer "B.Cu") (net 8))
 (segment (start 69.0183 74.7931) (end 68.1578 73.9326) (width 0.25) (layer "B.Cu") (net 8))
 (segment (start 73.606 72.2429) (end 77.5631 76.2) (width 0.25) (layer "B.Cu") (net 8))
 (segment (start 68.1578 72.9) (end 68.8149 72.2429) (width 0.25) (layer "B.Cu") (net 8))
 (segment (start 69.3 75.92) (end 69.3 74.7931) (width 0.25) (layer "B.Cu") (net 8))
 (segment (start 77.5631 76.2) (end 78.74 76.2) (width 0.25) (layer "B.Cu") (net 8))
 (segment (start 69.3 74.7931) (end 69.0183 74.7931) (width 0.25) (layer "B.Cu") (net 8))
 (segment (start 78.74 76.2) (end 83.82 76.2) (width 0.25) (layer "B.Cu") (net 8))
 (segment (start 68.1578 73.9326) (end 68.1578 72.9) (width 0.25) (layer "B.Cu") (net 8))
 (segment (start 69.3 73.38) (end 70.4269 73.38) (width 0.25) (layer "B.Cu") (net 7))
 (segment (start 75.7869 78.74) (end 78.74 78.74) (width 0.25) (layer "B.Cu") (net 7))
 (segment (start 70.4269 73.38) (end 75.7869 78.74) (width 0.25) (layer "B.Cu") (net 7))
 (segment (start 78.74 78.74) (end 83.82 78.74) (width 0.25) (layer "B.Cu") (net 7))
 (segment (start 83.82 81.28) (end 78.74 81.28) (width 0.25) (layer "B.Cu") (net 6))
 (segment (start 67.6905 78.4725) (end 68.9495 79.7315) (width 0.25) (layer "B.Cu") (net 6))
 (segment (start 67.6905 72.4495) (end 67.6905 78.4725) (width 0.25) (layer "B.Cu") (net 6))
 (segment (start 69.3 70.84) (end 67.6905 72.4495) (width 0.25) (layer "B.Cu") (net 6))
 (segment (start 77.5631 81.28) (end 78.74 81.28) (width 0.25) (layer "B.Cu") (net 6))
 (segment (start 68.9495 79.7315) (end 76.0146 79.7315) (width 0.25) (layer "B.Cu") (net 6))
 (segment (start 76.0146 79.7315) (end 77.5631 81.28) (width 0.25) (layer "B.Cu") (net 6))
 (segment (start 79.9169 86.912) (end 79.9169 70.5447) (width 0.25) (layer "F.Cu") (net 3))
 (segment (start 72.8572 51.9769) (end 73.66 51.9769) (width 0.25) (layer "F.Cu") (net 3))
 (segment (start 81.9049 88.9) (end 83.82 88.9) (width 0.25) (layer "F.Cu") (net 3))
 (segment (start 70.5246 62.0366) (end 71.8238 60.7374) (width 0.25) (layer "F.Cu") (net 3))
 (segment (start 79.2222 69.85) (end 78.338 69.85) (width 0.25) (layer "F.Cu") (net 3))
 (segment (start 70.4681 62.0931) (end 70.5246 62.0366) (width 0.25) (layer "F.Cu") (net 3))
 (segment (start 79.9169 70.5447) (end 79.2222 69.85) (width 0.25) (layer "F.Cu") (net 3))
 (segment (start 78.338 69.85) (end 70.5246 62.0366) (width 0.25) (layer "F.Cu") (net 3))
 (segment (start 79.1058 87.7231) (end 79.9169 86.912) (width 0.25) (layer "F.Cu") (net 3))
 (segment (start 69.3 62.0931) (end 70.4681 62.0931) (width 0.25) (layer "F.Cu") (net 3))
 (segment (start 73.66 51.9769) (end 73.66 50.8) (width 0.25) (layer "F.Cu") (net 3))
 (segment (start 79.9169 86.912) (end 81.9049 88.9) (width 0.25) (layer "F.Cu") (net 3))
 (segment (start 71.8238 53.0103) (end 72.8572 51.9769) (width 0.25) (layer "F.Cu") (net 3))
 (segment (start 69.3 63.22) (end 69.3 62.0931) (width 0.25) (layer "F.Cu") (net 3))
 (segment (start 78.74 87.7231) (end 79.1058 87.7231) (width 0.25) (layer "F.Cu") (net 3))
 (segment (start 71.8238 60.7374) (end 71.8238 53.0103) (width 0.25) (layer "F.Cu") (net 3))
 (segment (start 78.74 88.9) (end 78.74 87.7231) (width 0.25) (layer "F.Cu") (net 3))
 (segment (start 73.66 50.8) (end 63.66 50.8) (width 0.25) (layer "B.Cu") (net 3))
 (segment (start 63.66 50.8) (end 56.04 43.18) (width 0.25) (layer "B.Cu") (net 3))
 (segment (start 68.8063 82.1326) (end 61.04 74.3663) (width 0.25) (layer "F.Cu") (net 2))
 (segment (start 73.3357 82.1326) (end 68.8063 82.1326) (width 0.25) (layer "F.Cu") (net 2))
 (segment (start 77.5631 86.36) (end 73.3357 82.1326) (width 0.25) (layer "F.Cu") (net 2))
 (segment (start 61.04 74.3663) (end 61.04 43.18) (width 0.25) (layer "F.Cu") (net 2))
 (segment (start 78.74 86.36) (end 77.5631 86.36) (width 0.25) (layer "F.Cu") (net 2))
 (segment (start 78.74 86.36) (end 83.82 86.36) (width 0.25) (layer "B.Cu") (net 2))
 (segment (start 83.82 60.96) (end 83.82 59.7831) (width 0.25) (layer "F.Cu") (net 14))
 (segment (start 58.5401 43.0638) (end 58.5401 49.0576) (width 0.25) (layer "F.Cu") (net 14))
 (segment (start 52.9325 64.6325) (end 54.06 65.76) (width 0.25) (layer "F.Cu") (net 14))
 (segment (start 84.2821 49.53) (end 83.361 49.53) (width 0.25) (layer "F.Cu") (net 14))
 (segment (start 83.82 59.7831) (end 84.1878 59.7831) (width 0.25) (layer "F.Cu") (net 14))
 (segment (start 81.28 44.0463) (end 78.5572 41.3235) (width 0.25) (layer "F.Cu") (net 14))
 (segment (start 78.5572 41.3235) (end 60.2804 41.3235) (width 0.25) (layer "F.Cu") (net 14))
 (segment (start 58.5401 49.0576) (end 52.9325 54.6652) (width 0.25) (layer "F.Cu") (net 14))
 (segment (start 83.361 49.53) (end 81.28 47.449) (width 0.25) (layer "F.Cu") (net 14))
 (segment (start 84.1878 59.7831) (end 85.0092 58.9617) (width 0.25) (layer "F.Cu") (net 14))
 (segment (start 85.0092 50.2571) (end 84.2821 49.53) (width 0.25) (layer "F.Cu") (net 14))
 (segment (start 81.28 47.449) (end 81.28 44.0463) (width 0.25) (layer "F.Cu") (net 14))
 (segment (start 60.2804 41.3235) (end 58.5401 43.0638) (width 0.25) (layer "F.Cu") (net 14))
 (segment (start 52.9325 54.6652) (end 52.9325 64.6325) (width 0.25) (layer "F.Cu") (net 14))
 (segment (start 85.0092 58.9617) (end 85.0092 50.2571) (width 0.25) (layer "F.Cu") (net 14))
 (segment (start 78.74 60.96) (end 83.82 60.96) (width 0.25) (layer "B.Cu") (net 14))
 (segment (start 79.9169 48.26) (end 78.74 48.26) (width 0.25) (layer "B.Cu") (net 1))
 (segment (start 77.5631 48.1129) (end 73.9002 44.45) (width 0.25) (layer "B.Cu") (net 1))
 (segment (start 83.82 45.72) (end 82.4569 45.72) (width 0.25) (layer "B.Cu") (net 1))
 (segment (start 82.4569 45.72) (end 79.9169 48.26) (width 0.25) (layer "B.Cu") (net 1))
 (segment (start 77.5631 48.26) (end 77.5631 48.1129) (width 0.25) (layer "B.Cu") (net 1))
 (segment (start 67.8669 43.18) (end 66.04 43.18) (width 0.25) (layer "B.Cu") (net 1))
 (segment (start 73.9002 44.45) (end 69.1369 44.45) (width 0.25) (layer "B.Cu") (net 1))
 (segment (start 78.74 48.26) (end 77.5631 48.26) (width 0.25) (layer "B.Cu") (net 1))
 (segment (start 69.1369 44.45) (end 67.8669 43.18) (width 0.25) (layer "B.Cu") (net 1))
 (segment (start 78.74 45.72) (end 79.9169 45.72) (width 0.25) (layer "B.Cu") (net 20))
 (segment (start 82.4569 43.18) (end 83.82 43.18) (width 0.25) (layer "B.Cu") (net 20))
 (segment (start 74.6869 43.18) (end 77.2269 45.72) (width 0.25) (layer "B.Cu") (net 20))
 (segment (start 77.2269 45.72) (end 78.74 45.72) (width 0.25) (layer "B.Cu") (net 20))
 (segment (start 73.66 43.18) (end 74.6869 43.18) (width 0.25) (layer "B.Cu") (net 20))
 (segment (start 79.9169 45.72) (end 82.4569 43.18) (width 0.25) (layer "B.Cu") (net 20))
 (segment (start 73.66 53.34) (end 73.66 52.1631) (width 0.25) (layer "B.Cu") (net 21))
 (segment (start 74.0278 52.1631) (end 74.8393 51.3516) (width 0.25) (layer "B.Cu") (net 21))
 (segment (start 73.66 52.1631) (end 74.0278 52.1631) (width 0.25) (layer "B.Cu") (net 21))
 (segment (start 74.8393 51.3516) (end 74.8393 46.8993) (width 0.25) (layer "B.Cu") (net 21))
 (segment (start 74.8393 46.8993) (end 73.66 45.72) (width 0.25) (layer "B.Cu") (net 21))
 (segment (start 70.0267 54.4462) (end 61.3711 54.4462) (width 0.25) (layer "B.Cu") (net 19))
 (segment (start 61.3711 54.4462) (end 56.4073 59.41) (width 0.25) (layer "B.Cu") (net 19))
 (segment (start 52.3762 60.7145) (end 52.3762 84.3962) (width 0.25) (layer "B.Cu") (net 19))
 (segment (start 75.4524 52.3974) (end 75.4524 53.7211) (width 0.25) (layer "B.Cu") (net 19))
 (segment (start 74.6273 54.5462) (end 70.1267 54.5462) (width 0.25) (layer "B.Cu") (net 19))
 (segment (start 56.4073 59.41) (end 53.6807 59.41) (width 0.25) (layer "B.Cu") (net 19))
 (segment (start 75.4524 53.7211) (end 74.6273 54.5462) (width 0.25) (layer "B.Cu") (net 19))
 (segment (start 78.4129 49.4369) (end 75.4524 52.3974) (width 0.25) (layer "B.Cu") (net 19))
 (segment (start 83.82 48.26) (end 82.6431 48.26) (width 0.25) (layer "B.Cu") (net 19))
 (segment (start 82.6431 48.26) (end 81.4662 49.4369) (width 0.25) (layer "B.Cu") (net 19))
 (segment (start 70.1267 54.5462) (end 70.0267 54.4462) (width 0.25) (layer "B.Cu") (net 19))
 (segment (start 52.3762 84.3962) (end 54.06 86.08) (width 0.25) (layer "B.Cu") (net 19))
 (segment (start 81.4662 49.4369) (end 78.4129 49.4369) (width 0.25) (layer "B.Cu") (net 19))
 (segment (start 53.6807 59.41) (end 52.3762 60.7145) (width 0.25) (layer "B.Cu") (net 19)))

